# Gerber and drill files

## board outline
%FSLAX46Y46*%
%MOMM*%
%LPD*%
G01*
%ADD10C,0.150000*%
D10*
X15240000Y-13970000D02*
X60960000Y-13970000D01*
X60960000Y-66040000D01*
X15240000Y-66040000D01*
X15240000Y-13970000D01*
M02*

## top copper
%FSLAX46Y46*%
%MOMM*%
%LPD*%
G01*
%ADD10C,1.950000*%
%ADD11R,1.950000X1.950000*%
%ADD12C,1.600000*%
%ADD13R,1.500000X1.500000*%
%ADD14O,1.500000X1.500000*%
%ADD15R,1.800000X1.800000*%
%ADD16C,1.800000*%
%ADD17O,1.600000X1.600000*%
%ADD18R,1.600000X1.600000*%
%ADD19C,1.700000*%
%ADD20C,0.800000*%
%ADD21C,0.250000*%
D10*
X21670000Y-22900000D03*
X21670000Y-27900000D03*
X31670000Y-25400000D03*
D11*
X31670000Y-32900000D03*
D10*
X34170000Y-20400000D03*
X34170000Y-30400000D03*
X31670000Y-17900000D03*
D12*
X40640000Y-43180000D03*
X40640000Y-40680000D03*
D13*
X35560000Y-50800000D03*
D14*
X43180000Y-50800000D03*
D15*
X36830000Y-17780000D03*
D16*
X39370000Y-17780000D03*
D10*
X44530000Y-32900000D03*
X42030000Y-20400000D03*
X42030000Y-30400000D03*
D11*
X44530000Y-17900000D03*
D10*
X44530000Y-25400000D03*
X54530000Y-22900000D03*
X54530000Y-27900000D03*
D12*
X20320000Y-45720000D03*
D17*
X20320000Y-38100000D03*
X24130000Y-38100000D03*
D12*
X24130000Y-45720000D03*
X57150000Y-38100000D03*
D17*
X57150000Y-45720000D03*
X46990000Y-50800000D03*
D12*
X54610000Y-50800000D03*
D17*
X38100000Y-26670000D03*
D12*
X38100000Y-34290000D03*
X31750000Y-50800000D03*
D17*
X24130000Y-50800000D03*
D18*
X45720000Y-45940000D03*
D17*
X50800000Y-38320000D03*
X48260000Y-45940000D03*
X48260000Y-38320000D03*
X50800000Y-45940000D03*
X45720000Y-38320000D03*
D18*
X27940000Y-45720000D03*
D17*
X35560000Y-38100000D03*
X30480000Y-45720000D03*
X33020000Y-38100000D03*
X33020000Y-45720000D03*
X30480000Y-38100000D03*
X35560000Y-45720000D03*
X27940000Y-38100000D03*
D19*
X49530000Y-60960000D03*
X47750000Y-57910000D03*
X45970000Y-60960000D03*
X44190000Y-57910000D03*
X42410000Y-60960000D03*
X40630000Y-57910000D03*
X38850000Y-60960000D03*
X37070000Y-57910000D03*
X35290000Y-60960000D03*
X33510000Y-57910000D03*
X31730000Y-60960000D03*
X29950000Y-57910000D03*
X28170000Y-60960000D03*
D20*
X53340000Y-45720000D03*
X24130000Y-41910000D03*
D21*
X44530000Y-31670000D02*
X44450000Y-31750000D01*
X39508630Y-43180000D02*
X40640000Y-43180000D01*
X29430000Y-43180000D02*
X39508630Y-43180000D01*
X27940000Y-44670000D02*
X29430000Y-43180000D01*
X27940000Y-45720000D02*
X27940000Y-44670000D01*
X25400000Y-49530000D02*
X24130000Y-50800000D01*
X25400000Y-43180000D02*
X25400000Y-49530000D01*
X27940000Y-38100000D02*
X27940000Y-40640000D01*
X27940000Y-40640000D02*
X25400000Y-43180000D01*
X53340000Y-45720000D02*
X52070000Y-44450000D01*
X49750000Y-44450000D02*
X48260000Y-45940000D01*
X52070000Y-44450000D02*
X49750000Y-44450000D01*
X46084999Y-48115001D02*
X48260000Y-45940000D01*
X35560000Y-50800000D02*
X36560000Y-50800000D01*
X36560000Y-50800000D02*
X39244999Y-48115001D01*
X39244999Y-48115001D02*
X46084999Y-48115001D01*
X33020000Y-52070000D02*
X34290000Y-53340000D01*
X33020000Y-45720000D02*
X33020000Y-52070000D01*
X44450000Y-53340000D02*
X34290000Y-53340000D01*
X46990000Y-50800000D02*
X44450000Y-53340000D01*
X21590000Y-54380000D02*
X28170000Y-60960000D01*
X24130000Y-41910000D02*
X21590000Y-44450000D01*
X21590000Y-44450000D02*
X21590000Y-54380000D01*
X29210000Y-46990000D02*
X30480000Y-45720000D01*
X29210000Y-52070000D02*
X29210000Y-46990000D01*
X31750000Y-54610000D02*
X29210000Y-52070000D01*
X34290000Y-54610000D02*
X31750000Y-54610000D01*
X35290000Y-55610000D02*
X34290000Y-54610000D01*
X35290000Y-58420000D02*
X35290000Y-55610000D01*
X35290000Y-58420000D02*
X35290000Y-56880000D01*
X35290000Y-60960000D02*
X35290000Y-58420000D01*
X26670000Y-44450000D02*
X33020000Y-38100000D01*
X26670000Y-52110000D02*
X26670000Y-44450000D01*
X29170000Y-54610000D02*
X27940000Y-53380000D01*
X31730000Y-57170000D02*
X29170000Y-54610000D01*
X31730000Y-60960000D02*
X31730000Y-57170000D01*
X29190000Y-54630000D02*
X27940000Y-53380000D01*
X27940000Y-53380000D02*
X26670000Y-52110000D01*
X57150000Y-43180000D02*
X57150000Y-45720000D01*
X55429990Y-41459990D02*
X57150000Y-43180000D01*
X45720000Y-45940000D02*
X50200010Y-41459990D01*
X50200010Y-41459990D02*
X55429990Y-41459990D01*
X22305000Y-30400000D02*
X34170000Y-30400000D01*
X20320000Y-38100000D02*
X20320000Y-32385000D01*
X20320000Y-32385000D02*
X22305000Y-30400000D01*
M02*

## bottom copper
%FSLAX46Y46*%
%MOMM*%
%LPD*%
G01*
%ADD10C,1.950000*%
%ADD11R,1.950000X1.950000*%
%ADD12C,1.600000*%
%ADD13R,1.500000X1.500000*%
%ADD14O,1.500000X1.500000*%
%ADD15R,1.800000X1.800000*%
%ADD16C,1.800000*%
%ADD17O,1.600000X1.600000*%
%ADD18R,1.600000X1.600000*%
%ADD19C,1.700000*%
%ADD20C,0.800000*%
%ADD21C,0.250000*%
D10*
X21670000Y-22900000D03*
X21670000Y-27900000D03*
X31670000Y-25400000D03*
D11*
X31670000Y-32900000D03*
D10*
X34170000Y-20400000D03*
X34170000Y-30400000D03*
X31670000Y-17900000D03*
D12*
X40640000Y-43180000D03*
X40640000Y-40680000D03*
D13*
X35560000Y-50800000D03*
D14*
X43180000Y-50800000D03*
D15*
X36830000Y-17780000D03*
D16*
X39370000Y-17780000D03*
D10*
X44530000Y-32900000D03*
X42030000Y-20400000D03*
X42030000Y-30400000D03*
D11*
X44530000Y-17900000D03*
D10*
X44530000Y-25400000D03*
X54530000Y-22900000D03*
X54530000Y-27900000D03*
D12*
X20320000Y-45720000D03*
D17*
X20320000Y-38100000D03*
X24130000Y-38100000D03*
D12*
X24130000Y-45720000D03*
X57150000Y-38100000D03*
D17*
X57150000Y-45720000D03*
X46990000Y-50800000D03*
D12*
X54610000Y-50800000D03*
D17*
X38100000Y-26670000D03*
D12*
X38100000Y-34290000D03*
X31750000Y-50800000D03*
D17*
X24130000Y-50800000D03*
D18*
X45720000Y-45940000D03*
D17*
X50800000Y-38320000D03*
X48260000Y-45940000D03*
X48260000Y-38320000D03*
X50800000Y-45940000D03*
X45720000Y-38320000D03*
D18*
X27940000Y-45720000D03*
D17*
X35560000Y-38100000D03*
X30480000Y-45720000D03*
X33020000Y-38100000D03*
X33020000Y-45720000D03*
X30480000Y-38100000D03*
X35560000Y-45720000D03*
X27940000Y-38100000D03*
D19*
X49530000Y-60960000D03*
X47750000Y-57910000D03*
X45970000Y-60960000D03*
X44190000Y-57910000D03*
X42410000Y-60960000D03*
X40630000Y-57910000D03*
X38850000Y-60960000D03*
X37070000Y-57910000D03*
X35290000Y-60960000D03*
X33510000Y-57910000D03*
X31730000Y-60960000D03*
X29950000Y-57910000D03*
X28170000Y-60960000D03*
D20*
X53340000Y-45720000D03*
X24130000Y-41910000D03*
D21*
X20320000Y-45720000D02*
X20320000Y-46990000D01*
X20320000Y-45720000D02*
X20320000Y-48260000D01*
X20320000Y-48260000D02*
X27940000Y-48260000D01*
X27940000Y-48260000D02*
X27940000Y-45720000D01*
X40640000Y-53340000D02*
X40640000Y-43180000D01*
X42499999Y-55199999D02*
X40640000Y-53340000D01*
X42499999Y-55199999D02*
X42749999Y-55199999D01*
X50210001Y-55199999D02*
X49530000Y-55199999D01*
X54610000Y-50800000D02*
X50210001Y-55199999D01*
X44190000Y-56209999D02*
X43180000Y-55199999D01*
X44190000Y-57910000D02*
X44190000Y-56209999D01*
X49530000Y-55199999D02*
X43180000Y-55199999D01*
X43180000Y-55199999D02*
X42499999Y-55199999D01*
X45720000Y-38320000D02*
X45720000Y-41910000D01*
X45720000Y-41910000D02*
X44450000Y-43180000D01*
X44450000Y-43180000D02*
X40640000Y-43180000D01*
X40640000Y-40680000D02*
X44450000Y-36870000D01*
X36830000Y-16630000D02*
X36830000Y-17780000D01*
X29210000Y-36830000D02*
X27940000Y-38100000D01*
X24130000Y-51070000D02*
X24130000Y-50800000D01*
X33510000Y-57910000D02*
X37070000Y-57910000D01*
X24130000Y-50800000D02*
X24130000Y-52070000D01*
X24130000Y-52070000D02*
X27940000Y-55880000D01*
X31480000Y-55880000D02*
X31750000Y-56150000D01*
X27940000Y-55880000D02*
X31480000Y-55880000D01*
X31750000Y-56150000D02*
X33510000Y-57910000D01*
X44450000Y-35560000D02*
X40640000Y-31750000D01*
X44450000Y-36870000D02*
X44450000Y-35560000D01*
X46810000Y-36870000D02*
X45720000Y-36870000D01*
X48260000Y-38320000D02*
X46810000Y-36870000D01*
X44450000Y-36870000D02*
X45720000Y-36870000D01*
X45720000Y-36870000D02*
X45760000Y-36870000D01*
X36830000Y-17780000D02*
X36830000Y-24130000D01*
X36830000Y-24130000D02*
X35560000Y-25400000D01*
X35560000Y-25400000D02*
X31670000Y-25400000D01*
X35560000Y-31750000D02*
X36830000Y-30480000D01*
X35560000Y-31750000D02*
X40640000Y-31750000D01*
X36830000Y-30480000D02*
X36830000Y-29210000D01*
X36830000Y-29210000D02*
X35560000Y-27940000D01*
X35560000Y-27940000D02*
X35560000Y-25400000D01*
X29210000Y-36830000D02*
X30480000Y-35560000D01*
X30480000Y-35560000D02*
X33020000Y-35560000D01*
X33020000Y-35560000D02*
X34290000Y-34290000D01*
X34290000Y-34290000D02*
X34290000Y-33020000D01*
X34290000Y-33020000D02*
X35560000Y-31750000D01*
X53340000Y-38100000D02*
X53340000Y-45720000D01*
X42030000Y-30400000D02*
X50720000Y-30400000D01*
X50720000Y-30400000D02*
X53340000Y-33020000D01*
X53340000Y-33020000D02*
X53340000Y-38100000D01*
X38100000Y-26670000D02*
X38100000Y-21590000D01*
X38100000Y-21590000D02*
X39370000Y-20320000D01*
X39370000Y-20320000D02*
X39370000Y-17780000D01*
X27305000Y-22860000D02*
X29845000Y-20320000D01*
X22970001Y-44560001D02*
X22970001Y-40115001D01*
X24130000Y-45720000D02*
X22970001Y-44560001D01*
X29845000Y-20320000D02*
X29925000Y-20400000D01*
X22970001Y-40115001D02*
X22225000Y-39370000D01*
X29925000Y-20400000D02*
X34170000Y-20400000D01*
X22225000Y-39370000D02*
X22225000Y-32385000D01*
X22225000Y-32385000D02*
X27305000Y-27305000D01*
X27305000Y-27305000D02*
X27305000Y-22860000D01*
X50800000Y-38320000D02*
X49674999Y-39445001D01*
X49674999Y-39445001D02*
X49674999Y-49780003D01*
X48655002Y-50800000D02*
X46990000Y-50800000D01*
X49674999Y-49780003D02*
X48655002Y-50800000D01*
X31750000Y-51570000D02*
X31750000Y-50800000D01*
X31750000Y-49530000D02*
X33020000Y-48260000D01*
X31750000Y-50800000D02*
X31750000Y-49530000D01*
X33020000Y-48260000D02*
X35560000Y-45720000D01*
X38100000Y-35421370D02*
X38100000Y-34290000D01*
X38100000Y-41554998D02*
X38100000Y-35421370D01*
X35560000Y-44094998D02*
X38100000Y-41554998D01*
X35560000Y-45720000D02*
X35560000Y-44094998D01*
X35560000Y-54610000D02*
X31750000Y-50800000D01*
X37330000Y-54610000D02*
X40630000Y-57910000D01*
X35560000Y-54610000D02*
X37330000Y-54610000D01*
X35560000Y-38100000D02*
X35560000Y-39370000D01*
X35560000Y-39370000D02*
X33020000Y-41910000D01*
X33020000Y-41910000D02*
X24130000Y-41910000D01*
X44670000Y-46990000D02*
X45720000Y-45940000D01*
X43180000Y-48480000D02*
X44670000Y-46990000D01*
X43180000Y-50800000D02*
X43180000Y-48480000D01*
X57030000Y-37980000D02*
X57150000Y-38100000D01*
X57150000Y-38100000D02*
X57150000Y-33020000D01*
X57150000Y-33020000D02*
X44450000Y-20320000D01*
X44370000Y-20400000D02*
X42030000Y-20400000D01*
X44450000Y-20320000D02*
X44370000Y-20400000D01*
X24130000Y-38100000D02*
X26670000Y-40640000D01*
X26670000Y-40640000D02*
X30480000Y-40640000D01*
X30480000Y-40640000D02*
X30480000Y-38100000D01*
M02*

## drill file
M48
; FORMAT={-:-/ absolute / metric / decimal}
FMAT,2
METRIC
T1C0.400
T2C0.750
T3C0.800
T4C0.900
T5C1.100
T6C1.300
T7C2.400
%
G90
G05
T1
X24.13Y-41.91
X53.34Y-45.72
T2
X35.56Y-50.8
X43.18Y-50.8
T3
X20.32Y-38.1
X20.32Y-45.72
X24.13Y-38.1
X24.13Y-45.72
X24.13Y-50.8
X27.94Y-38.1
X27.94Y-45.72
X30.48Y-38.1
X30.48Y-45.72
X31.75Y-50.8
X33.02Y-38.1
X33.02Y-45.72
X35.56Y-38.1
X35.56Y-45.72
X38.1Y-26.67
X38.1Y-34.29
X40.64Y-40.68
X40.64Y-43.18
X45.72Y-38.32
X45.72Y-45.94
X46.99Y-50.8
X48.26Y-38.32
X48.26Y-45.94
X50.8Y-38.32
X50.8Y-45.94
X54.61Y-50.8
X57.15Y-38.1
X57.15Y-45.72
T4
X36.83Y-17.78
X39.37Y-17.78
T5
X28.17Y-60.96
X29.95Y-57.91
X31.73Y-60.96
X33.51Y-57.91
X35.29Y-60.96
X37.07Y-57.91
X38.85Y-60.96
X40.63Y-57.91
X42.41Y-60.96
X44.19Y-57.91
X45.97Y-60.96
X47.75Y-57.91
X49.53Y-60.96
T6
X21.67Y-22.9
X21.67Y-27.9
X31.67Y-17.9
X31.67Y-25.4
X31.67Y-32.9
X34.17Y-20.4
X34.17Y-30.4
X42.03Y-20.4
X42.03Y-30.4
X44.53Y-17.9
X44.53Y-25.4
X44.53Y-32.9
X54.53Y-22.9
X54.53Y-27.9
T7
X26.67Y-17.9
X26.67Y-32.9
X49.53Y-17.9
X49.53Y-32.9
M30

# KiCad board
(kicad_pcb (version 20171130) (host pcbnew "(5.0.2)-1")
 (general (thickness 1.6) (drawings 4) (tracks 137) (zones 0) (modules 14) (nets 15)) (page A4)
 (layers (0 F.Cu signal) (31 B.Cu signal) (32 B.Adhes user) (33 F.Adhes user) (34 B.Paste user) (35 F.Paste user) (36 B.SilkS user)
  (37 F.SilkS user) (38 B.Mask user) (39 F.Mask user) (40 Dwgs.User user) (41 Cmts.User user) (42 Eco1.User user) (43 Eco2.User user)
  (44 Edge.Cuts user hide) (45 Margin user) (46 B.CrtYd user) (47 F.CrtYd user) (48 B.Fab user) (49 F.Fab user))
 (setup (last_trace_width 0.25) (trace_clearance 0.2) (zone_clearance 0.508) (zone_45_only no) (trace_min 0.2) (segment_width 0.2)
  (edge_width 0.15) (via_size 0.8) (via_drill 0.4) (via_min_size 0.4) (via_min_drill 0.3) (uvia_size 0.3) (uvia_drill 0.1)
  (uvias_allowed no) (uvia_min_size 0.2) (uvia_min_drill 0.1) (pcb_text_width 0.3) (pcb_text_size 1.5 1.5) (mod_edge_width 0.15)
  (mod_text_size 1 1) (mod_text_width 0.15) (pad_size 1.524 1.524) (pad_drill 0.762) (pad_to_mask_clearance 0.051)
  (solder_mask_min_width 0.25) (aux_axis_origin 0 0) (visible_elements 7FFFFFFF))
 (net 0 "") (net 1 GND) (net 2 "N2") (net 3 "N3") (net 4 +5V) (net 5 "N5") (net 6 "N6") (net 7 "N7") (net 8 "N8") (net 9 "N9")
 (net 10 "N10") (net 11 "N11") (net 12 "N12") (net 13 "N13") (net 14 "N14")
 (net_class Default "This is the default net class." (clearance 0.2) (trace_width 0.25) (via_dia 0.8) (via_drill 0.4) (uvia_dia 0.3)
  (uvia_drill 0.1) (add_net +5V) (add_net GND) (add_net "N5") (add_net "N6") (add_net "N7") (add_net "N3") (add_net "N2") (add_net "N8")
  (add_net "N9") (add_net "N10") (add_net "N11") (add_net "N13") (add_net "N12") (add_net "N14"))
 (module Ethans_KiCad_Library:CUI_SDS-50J (layer F.Cu) (at 26.67 25.4 270)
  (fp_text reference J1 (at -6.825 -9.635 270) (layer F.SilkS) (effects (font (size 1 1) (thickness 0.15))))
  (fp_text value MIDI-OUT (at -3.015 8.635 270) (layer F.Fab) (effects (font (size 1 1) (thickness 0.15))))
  (pad E1 thru_hole circle (at -2.5 5 270) (size 1.95 1.95) (drill 1.3) (layers *.Cu *.Mask))
  (pad E2 thru_hole circle (at 2.5 5 270) (size 1.95 1.95) (drill 1.3) (layers *.Cu *.Mask))
  (pad 2 thru_hole circle (at 0 -5 270) (size 1.95 1.95) (drill 1.3) (layers *.Cu *.Mask) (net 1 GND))
  (pad 1 thru_hole rect (at 7.5 -5 270) (size 1.95 1.95) (drill 1.3) (layers *.Cu *.Mask))
  (pad 5 thru_hole circle (at -5 -7.5 270) (size 1.95 1.95) (drill 1.3) (layers *.Cu *.Mask) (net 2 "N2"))
  (pad 4 thru_hole circle (at 5 -7.5 270) (size 1.95 1.95) (drill 1.3) (layers *.Cu *.Mask) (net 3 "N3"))
  (pad None np_thru_hole circle (at 7.5 0 270) (size 2.4 2.4) (drill 2.4) (layers *.Cu *.Mask))
  (pad None np_thru_hole circle (at -7.5 0 270) (size 2.4 2.4) (drill 2.4) (layers *.Cu *.Mask))
  (pad 3 thru_hole circle (at -7.5 -5 270) (size 1.95 1.95) (drill 1.3) (layers *.Cu *.Mask)))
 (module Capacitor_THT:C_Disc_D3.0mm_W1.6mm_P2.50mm (layer F.Cu) (at 40.64 43.18 90)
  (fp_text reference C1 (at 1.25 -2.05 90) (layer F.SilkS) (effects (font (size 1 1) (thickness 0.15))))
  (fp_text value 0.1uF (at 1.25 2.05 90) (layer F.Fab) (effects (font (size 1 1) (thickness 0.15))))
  (pad 1 thru_hole circle (at 0 0 90) (size 1.6 1.6) (drill 0.8) (layers *.Cu *.Mask) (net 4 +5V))
  (pad 2 thru_hole circle (at 2.5 0 90) (size 1.6 1.6) (drill 0.8) (layers *.Cu *.Mask) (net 1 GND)))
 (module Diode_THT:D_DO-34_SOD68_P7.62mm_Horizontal (layer F.Cu) (at 35.56 50.8)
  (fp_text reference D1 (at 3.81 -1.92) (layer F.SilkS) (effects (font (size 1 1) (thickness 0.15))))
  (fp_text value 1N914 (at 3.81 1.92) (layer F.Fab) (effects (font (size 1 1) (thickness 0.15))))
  (pad 1 thru_hole rect (at 0 0) (size 1.5 1.5) (drill 0.75) (layers *.Cu *.Mask) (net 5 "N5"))
  (pad 2 thru_hole oval (at 7.62 0) (size 1.5 1.5) (drill 0.75) (layers *.Cu *.Mask) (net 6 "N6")))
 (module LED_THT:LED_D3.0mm (layer F.Cu) (at 36.83 17.78)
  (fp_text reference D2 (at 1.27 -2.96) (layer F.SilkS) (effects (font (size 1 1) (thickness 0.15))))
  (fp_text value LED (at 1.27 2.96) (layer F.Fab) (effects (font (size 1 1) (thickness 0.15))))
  (pad 1 thru_hole rect (at 0 0) (size 1.8 1.8) (drill 0.9) (layers *.Cu *.Mask) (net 1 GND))
  (pad 2 thru_hole circle (at 2.54 0) (size 1.8 1.8) (drill 0.9) (layers *.Cu *.Mask) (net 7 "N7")))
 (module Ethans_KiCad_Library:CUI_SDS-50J (layer F.Cu) (at 49.53 25.4 90)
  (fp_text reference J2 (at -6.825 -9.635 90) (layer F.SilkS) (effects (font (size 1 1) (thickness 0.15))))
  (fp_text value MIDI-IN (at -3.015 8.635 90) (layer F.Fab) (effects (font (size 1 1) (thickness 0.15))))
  (pad 3 thru_hole circle (at -7.5 -5 90) (size 1.95 1.95) (drill 1.3) (layers *.Cu *.Mask))
  (pad None np_thru_hole circle (at -7.5 0 90) (size 2.4 2.4) (drill 2.4) (layers *.Cu *.Mask))
  (pad None np_thru_hole circle (at 7.5 0 90) (size 2.4 2.4) (drill 2.4) (layers *.Cu *.Mask))
  (pad 4 thru_hole circle (at 5 -7.5 90) (size 1.95 1.95) (drill 1.3) (layers *.Cu *.Mask) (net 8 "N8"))
  (pad 5 thru_hole circle (at -5 -7.5 90) (size 1.95 1.95) (drill 1.3) (layers *.Cu *.Mask) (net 5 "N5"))
  (pad 1 thru_hole rect (at 7.5 -5 90) (size 1.95 1.95) (drill 1.3) (layers *.Cu *.Mask))
  (pad 2 thru_hole circle (at 0 -5 90) (size 1.95 1.95) (drill 1.3) (layers *.Cu *.Mask))
  (pad E2 thru_hole circle (at 2.5 5 90) (size 1.95 1.95) (drill 1.3) (layers *.Cu *.Mask))
  (pad E1 thru_hole circle (at -2.5 5 90) (size 1.95 1.95) (drill 1.3) (layers *.Cu *.Mask)))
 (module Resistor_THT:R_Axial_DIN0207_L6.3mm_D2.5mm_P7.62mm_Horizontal (layer F.Cu) (at 20.32 45.72 90)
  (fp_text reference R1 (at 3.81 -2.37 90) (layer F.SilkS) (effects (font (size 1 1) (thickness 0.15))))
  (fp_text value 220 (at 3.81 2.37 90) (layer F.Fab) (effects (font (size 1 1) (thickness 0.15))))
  (pad 1 thru_hole circle (at 0 0 90) (size 1.6 1.6) (drill 0.8) (layers *.Cu *.Mask) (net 4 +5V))
  (pad 2 thru_hole oval (at 7.62 0 90) (size 1.6 1.6) (drill 0.8) (layers *.Cu *.Mask) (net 3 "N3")))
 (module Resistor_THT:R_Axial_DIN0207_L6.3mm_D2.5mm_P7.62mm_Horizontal (layer F.Cu) (at 24.13 45.72 90)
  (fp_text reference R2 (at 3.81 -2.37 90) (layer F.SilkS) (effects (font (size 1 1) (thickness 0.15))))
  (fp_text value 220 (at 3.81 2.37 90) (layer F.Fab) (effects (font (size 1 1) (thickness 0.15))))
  (pad 2 thru_hole oval (at 7.62 0 90) (size 1.6 1.6) (drill 0.8) (layers *.Cu *.Mask) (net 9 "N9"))
  (pad 1 thru_hole circle (at 0 0 90) (size 1.6 1.6) (drill 0.8) (layers *.Cu *.Mask) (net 2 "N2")))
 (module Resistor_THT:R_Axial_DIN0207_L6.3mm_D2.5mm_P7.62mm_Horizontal (layer F.Cu) (at 57.15 38.1 270)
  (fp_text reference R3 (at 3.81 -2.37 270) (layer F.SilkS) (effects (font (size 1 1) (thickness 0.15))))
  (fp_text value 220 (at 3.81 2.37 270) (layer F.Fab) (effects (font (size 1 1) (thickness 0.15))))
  (pad 1 thru_hole circle (at 0 0 270) (size 1.6 1.6) (drill 0.8) (layers *.Cu *.Mask) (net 8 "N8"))
  (pad 2 thru_hole oval (at 7.62 0 270) (size 1.6 1.6) (drill 0.8) (layers *.Cu *.Mask) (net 6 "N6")))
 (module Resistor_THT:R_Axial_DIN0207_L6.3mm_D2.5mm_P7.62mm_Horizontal (layer F.Cu) (at 54.61 50.8 180)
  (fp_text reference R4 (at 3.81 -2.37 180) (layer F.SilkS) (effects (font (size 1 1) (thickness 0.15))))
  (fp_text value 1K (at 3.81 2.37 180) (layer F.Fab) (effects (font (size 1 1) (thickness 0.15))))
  (pad 2 thru_hole oval (at 7.62 0 180) (size 1.6 1.6) (drill 0.8) (layers *.Cu *.Mask) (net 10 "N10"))
  (pad 1 thru_hole circle (at 0 0 180) (size 1.6 1.6) (drill 0.8) (layers *.Cu *.Mask) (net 4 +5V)))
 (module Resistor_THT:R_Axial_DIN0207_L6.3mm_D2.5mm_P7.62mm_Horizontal (layer F.Cu) (at 38.1 34.29 90)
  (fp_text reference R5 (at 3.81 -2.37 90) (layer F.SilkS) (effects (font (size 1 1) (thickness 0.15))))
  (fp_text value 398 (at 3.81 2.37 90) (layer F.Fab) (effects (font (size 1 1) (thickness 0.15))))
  (pad 2 thru_hole oval (at 7.62 0 90) (size 1.6 1.6) (drill 0.8) (layers *.Cu *.Mask) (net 7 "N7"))
  (pad 1 thru_hole circle (at 0 0 90) (size 1.6 1.6) (drill 0.8) (layers *.Cu *.Mask) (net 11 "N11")))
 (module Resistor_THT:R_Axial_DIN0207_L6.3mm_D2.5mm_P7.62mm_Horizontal (layer F.Cu) (at 31.75 50.8 180)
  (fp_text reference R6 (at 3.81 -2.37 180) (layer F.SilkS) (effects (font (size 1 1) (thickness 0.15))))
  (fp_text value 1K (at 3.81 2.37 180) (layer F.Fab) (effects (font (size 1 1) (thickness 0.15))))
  (pad 1 thru_hole circle (at 0 0 180) (size 1.6 1.6) (drill 0.8) (layers *.Cu *.Mask) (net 11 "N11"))
  (pad 2 thru_hole oval (at 7.62 0 180) (size 1.6 1.6) (drill 0.8) (layers *.Cu *.Mask) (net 1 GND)))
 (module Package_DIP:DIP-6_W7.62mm (layer F.Cu) (at 45.72 45.94 90)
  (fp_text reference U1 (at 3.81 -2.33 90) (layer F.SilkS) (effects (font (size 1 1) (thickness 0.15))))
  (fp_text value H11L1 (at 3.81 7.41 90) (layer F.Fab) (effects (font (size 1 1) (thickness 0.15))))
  (pad 1 thru_hole rect (at 0 0 90) (size 1.6 1.6) (drill 0.8) (layers *.Cu *.Mask) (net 6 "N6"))
  (pad 4 thru_hole oval (at 7.62 5.08 90) (size 1.6 1.6) (drill 0.8) (layers *.Cu *.Mask) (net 10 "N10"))
  (pad 2 thru_hole oval (at 0 2.54 90) (size 1.6 1.6) (drill 0.8) (layers *.Cu *.Mask) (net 5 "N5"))
  (pad 5 thru_hole oval (at 7.62 2.54 90) (size 1.6 1.6) (drill 0.8) (layers *.Cu *.Mask) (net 1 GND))
  (pad 3 thru_hole oval (at 0 5.08 90) (size 1.6 1.6) (drill 0.8) (layers *.Cu *.Mask))
  (pad 6 thru_hole oval (at 7.62 0 90) (size 1.6 1.6) (drill 0.8) (layers *.Cu *.Mask) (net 4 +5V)))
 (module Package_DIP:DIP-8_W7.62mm (layer F.Cu) (at 27.94 45.72 90)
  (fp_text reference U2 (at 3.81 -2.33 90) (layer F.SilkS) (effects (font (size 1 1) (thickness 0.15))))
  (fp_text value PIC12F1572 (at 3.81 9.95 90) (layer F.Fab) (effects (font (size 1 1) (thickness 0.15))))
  (pad 1 thru_hole rect (at 0 0 90) (size 1.6 1.6) (drill 0.8) (layers *.Cu *.Mask) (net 4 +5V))
  (pad 5 thru_hole oval (at 7.62 7.62 90) (size 1.6 1.6) (drill 0.8) (layers *.Cu *.Mask) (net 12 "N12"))
  (pad 2 thru_hole oval (at 0 2.54 90) (size 1.6 1.6) (drill 0.8) (layers *.Cu *.Mask) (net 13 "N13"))
  (pad 6 thru_hole oval (at 7.62 5.08 90) (size 1.6 1.6) (drill 0.8) (layers *.Cu *.Mask) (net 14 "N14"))
  (pad 3 thru_hole oval (at 0 5.08 90) (size 1.6 1.6) (drill 0.8) (layers *.Cu *.Mask) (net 10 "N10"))
  (pad 7 thru_hole oval (at 7.62 2.54 90) (size 1.6 1.6) (drill 0.8) (layers *.Cu *.Mask) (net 9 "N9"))
  (pad 4 thru_hole oval (at 0 7.62 90) (size 1.6 1.6) (drill 0.8) (layers *.Cu *.Mask) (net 11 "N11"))
  (pad 8 thru_hole oval (at 7.62 0 90) (size 1.6 1.6) (drill 0.8) (layers *.Cu *.Mask) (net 1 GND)))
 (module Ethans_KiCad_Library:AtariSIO (layer F.Cu) (at 35.29 64.01)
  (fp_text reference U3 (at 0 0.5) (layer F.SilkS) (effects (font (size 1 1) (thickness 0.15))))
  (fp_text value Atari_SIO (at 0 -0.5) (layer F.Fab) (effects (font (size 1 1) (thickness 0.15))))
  (pad 13 thru_hole circle (at 14.24 -3.05) (size 1.7 1.7) (drill 1.1) (layers *.Cu *.Mask))
  (pad 12 thru_hole circle (at 12.46 -6.1) (size 1.7 1.7) (drill 1.1) (layers *.Cu *.Mask))
  (pad 11 thru_hole circle (at 10.68 -3.05) (size 1.7 1.7) (drill 1.1) (layers *.Cu *.Mask))
  (pad 10 thru_hole circle (at 8.9 -6.1) (size 1.7 1.7) (drill 1.1) (layers *.Cu *.Mask) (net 4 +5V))
  (pad 9 thru_hole circle (at 7.12 -3.05) (size 1.7 1.7) (drill 1.1) (layers *.Cu *.Mask))
  (pad 8 thru_hole circle (at 5.34 -6.1) (size 1.7 1.7) (drill 1.1) (layers *.Cu *.Mask) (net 11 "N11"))
  (pad 7 thru_hole circle (at 3.56 -3.05) (size 1.7 1.7) (drill 1.1) (layers *.Cu *.Mask))
  (pad 6 thru_hole circle (at 1.78 -6.1) (size 1.7 1.7) (drill 1.1) (layers *.Cu *.Mask) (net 1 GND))
  (pad 5 thru_hole circle (at 0 -3.05) (size 1.7 1.7) (drill 1.1) (layers *.Cu *.Mask) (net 13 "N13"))
  (pad 4 thru_hole circle (at -1.78 -6.1) (size 1.7 1.7) (drill 1.1) (layers *.Cu *.Mask) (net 1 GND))
  (pad 3 thru_hole circle (at -3.56 -3.05) (size 1.7 1.7) (drill 1.1) (layers *.Cu *.Mask) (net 14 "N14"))
  (pad 2 thru_hole circle (at -5.34 -6.1) (size 1.7 1.7) (drill 1.1) (layers *.Cu *.Mask))
  (pad 1 thru_hole circle (at -7.12 -3.05) (size 1.7 1.7) (drill 1.1) (layers *.Cu *.Mask) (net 12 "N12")))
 (gr_poly (pts (xy 15.24 13.97) (xy 60.96 13.97) (xy 60.96 66.04) (xy 15.24 66.04)) (layer Edge.Cuts) (width 0.15))
 (segment (start 44.53 31.67) (end 44.45 31.75) (width 0.25) (layer F.Cu) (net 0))
 (segment (start 20.32 45.72) (end 20.32 46.99) (width 0.25) (layer B.Cu) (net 4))
 (segment (start 20.32 45.72) (end 20.32 48.26) (width 0.25) (layer B.Cu) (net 4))
 (segment (start 20.32 48.26) (end 27.94 48.26) (width 0.25) (layer B.Cu) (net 4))
 (segment (start 27.94 48.26) (end 27.94 45.72) (width 0.25) (layer B.Cu) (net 4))
 (segment (start 39.50863 43.18) (end 40.64 43.18) (width 0.25) (layer F.Cu) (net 4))
 (segment (start 29.43 43.18) (end 39.50863 43.18) (width 0.25) (layer F.Cu) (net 4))
 (segment (start 27.94 44.67) (end 29.43 43.18) (width 0.25) (layer F.Cu) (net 4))
 (segment (start 27.94 45.72) (end 27.94 44.67) (width 0.25) (layer F.Cu) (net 4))
 (segment (start 40.64 53.34) (end 40.64 43.18) (width 0.25) (layer B.Cu) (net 4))
 (segment (start 42.499999 55.199999) (end 40.64 53.34) (width 0.25) (layer B.Cu) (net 4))
 (segment (start 42.499999 55.199999) (end 42.749999 55.199999) (width 0.25) (layer B.Cu) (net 4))
 (segment (start 50.210001 55.199999) (end 49.53 55.199999) (width 0.25) (layer B.Cu) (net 4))
 (segment (start 54.61 50.8) (end 50.210001 55.199999) (width 0.25) (layer B.Cu) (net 4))
 (segment (start 44.19 56.209999) (end 43.18 55.199999) (width 0.25) (layer B.Cu) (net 4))
 (segment (start 44.19 57.91) (end 44.19 56.209999) (width 0.25) (layer B.Cu) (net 4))
 (segment (start 49.53 55.199999) (end 43.18 55.199999) (width 0.25) (layer B.Cu) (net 4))
 (segment (start 43.18 55.199999) (end 42.499999 55.199999) (width 0.25) (layer B.Cu) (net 4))
 (segment (start 45.72 38.32) (end 45.72 41.91) (width 0.25) (layer B.Cu) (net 4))
 (segment (start 45.72 41.91) (end 44.45 43.18) (width 0.25) (layer B.Cu) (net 4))
 (segment (start 44.45 43.18) (end 40.64 43.18) (width 0.25) (layer B.Cu) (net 4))
 (segment (start 40.64 40.68) (end 44.45 36.87) (width 0.25) (layer B.Cu) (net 1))
 (segment (start 36.83 16.63) (end 36.83 17.78) (width 0.25) (layer B.Cu) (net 1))
 (segment (start 29.21 36.83) (end 27.94 38.1) (width 0.25) (layer B.Cu) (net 1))
 (segment (start 24.13 51.07) (end 24.13 50.8) (width 0.25) (layer B.Cu) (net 1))
 (segment (start 33.51 57.91) (end 37.07 57.91) (width 0.25) (layer B.Cu) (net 1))
 (segment (start 25.4 49.53) (end 24.13 50.8) (width 0.25) (layer F.Cu) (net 1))
 (segment (start 25.4 43.18) (end 25.4 49.53) (width 0.25) (layer F.Cu) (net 1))
 (segment (start 27.94 38.1) (end 27.94 40.64) (width 0.25) (layer F.Cu) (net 1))
 (segment (start 27.94 40.64) (end 25.4 43.18) (width 0.25) (layer F.Cu) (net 1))
 (segment (start 24.13 50.8) (end 24.13 52.07) (width 0.25) (layer B.Cu) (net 1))
 (segment (start 24.13 52.07) (end 27.94 55.88) (width 0.25) (layer B.Cu) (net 1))
 (segment (start 31.48 55.88) (end 31.75 56.15) (width 0.25) (layer B.Cu) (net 1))
 (segment (start 27.94 55.88) (end 31.48 55.88) (width 0.25) (layer B.Cu) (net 1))
 (segment (start 31.75 56.15) (end 33.51 57.91) (width 0.25) (layer B.Cu) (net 1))
 (segment (start 44.45 35.56) (end 40.64 31.75) (width 0.25) (layer B.Cu) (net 1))
 (segment (start 44.45 36.87) (end 44.45 35.56) (width 0.25) (layer B.Cu) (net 1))
 (segment (start 46.81 36.87) (end 45.72 36.87) (width 0.25) (layer B.Cu) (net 1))
 (segment (start 48.26 38.32) (end 46.81 36.87) (width 0.25) (layer B.Cu) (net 1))
 (segment (start 44.45 36.87) (end 45.72 36.87) (width 0.25) (layer B.Cu) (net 1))
 (segment (start 45.72 36.87) (end 45.76 36.87) (width 0.25) (layer B.Cu) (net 1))
 (segment (start 36.83 17.78) (end 36.83 24.13) (width 0.25) (layer B.Cu) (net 1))
 (segment (start 36.83 24.13) (end 35.56 25.4) (width 0.25) (layer B.Cu) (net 1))
 (segment (start 35.56 25.4) (end 31.67 25.4) (width 0.25) (layer B.Cu) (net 1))
 (segment (start 35.56 31.75) (end 36.83 30.48) (width 0.25) (layer B.Cu) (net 1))
 (segment (start 35.56 31.75) (end 40.64 31.75) (width 0.25) (layer B.Cu) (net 1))
 (segment (start 36.83 30.48) (end 36.83 29.21) (width 0.25) (layer B.Cu) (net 1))
 (segment (start 36.83 29.21) (end 35.56 27.94) (width 0.25) (layer B.Cu) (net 1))
 (segment (start 35.56 27.94) (end 35.56 25.4) (width 0.25) (layer B.Cu) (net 1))
 (segment (start 29.21 36.83) (end 30.48 35.56) (width 0.25) (layer B.Cu) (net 1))
 (segment (start 30.48 35.56) (end 33.02 35.56) (width 0.25) (layer B.Cu) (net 1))
 (segment (start 33.02 35.56) (end 34.29 34.29) (width 0.25) (layer B.Cu) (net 1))
 (segment (start 34.29 34.29) (end 34.29 33.02) (width 0.25) (layer B.Cu) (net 1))
 (segment (start 34.29 33.02) (end 35.56 31.75) (width 0.25) (layer B.Cu) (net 1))
 (segment (start 53.34 38.1) (end 53.34 45.72) (width 0.25) (layer B.Cu) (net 5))
 (via (at 53.34 45.72) (size 0.8) (drill 0.4) (layers F.Cu B.Cu) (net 5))
 (segment (start 53.34 45.72) (end 52.07 44.45) (width 0.25) (layer F.Cu) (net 5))
 (segment (start 49.75 44.45) (end 48.26 45.94) (width 0.25) (layer F.Cu) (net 5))
 (segment (start 52.07 44.45) (end 49.75 44.45) (width 0.25) (layer F.Cu) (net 5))
 (segment (start 46.084999 48.115001) (end 48.26 45.94) (width 0.25) (layer F.Cu) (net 5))
 (segment (start 35.56 50.8) (end 36.56 50.8) (width 0.25) (layer F.Cu) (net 5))
 (segment (start 36.56 50.8) (end 39.244999 48.115001) (width 0.25) (layer F.Cu) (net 5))
 (segment (start 39.244999 48.115001) (end 46.084999 48.115001) (width 0.25) (layer F.Cu) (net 5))
 (segment (start 42.03 30.4) (end 50.72 30.4) (width 0.25) (layer B.Cu) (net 5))
 (segment (start 50.72 30.4) (end 53.34 33.02) (width 0.25) (layer B.Cu) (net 5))
 (segment (start 53.34 33.02) (end 53.34 38.1) (width 0.25) (layer B.Cu) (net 5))
 (segment (start 38.1 26.67) (end 38.1 21.59) (width 0.25) (layer B.Cu) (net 7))
 (segment (start 38.1 21.59) (end 39.37 20.32) (width 0.25) (layer B.Cu) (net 7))
 (segment (start 39.37 20.32) (end 39.37 17.78) (width 0.25) (layer B.Cu) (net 7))
 (segment (start 27.305 22.86) (end 29.845 20.32) (width 0.25) (layer B.Cu) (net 2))
 (segment (start 22.970001 44.560001) (end 22.970001 40.115001) (width 0.25) (layer B.Cu) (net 2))
 (segment (start 24.13 45.72) (end 22.970001 44.560001) (width 0.25) (layer B.Cu) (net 2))
 (segment (start 29.845 20.32) (end 29.925 20.4) (width 0.25) (layer B.Cu) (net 2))
 (segment (start 22.970001 40.115001) (end 22.225 39.37) (width 0.25) (layer B.Cu) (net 2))
 (segment (start 29.925 20.4) (end 34.17 20.4) (width 0.25) (layer B.Cu) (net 2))
 (segment (start 22.225 39.37) (end 22.225 32.385) (width 0.25) (layer B.Cu) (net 2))
 (segment (start 22.225 32.385) (end 27.305 27.305) (width 0.25) (layer B.Cu) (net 2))
 (segment (start 27.305 27.305) (end 27.305 22.86) (width 0.25) (layer B.Cu) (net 2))
 (segment (start 33.02 52.07) (end 34.29 53.34) (width 0.25) (layer F.Cu) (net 10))
 (segment (start 50.8 38.32) (end 49.674999 39.445001) (width 0.25) (layer B.Cu) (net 10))
 (segment (start 49.674999 39.445001) (end 49.674999 49.780003) (width 0.25) (layer B.Cu) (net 10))
 (segment (start 33.02 45.72) (end 33.02 52.07) (width 0.25) (layer F.Cu) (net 10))
 (segment (start 44.45 53.34) (end 34.29 53.34) (width 0.25) (layer F.Cu) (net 10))
 (segment (start 46.99 50.8) (end 44.45 53.34) (width 0.25) (layer F.Cu) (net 10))
 (segment (start 48.655002 50.8) (end 46.99 50.8) (width 0.25) (layer B.Cu) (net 10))
 (segment (start 49.674999 49.780003) (end 48.655002 50.8) (width 0.25) (layer B.Cu) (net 10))
 (segment (start 31.75 51.57) (end 31.75 50.8) (width 0.25) (layer B.Cu) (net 11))
 (segment (start 31.75 49.53) (end 33.02 48.26) (width 0.25) (layer B.Cu) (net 11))
 (segment (start 31.75 50.8) (end 31.75 49.53) (width 0.25) (layer B.Cu) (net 11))
 (segment (start 33.02 48.26) (end 35.56 45.72) (width 0.25) (layer B.Cu) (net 11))
 (segment (start 38.1 35.42137) (end 38.1 34.29) (width 0.25) (layer B.Cu) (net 11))
 (segment (start 38.1 41.554998) (end 38.1 35.42137) (width 0.25) (layer B.Cu) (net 11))
 (segment (start 35.56 44.094998) (end 38.1 41.554998) (width 0.25) (layer B.Cu) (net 11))
 (segment (start 35.56 45.72) (end 35.56 44.094998) (width 0.25) (layer B.Cu) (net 11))
 (segment (start 35.56 54.61) (end 31.75 50.8) (width 0.25) (layer B.Cu) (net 11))
 (segment (start 37.33 54.61) (end 40.63 57.91) (width 0.25) (layer B.Cu) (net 11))
 (segment (start 35.56 54.61) (end 37.33 54.61) (width 0.25) (layer B.Cu) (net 11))
 (segment (start 35.56 38.1) (end 35.56 39.37) (width 0.25) (layer B.Cu) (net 12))
 (segment (start 35.56 39.37) (end 33.02 41.91) (width 0.25) (layer B.Cu) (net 12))
 (via (at 24.13 41.91) (size 0.8) (drill 0.4) (layers F.Cu B.Cu) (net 12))
 (segment (start 33.02 41.91) (end 24.13 41.91) (width 0.25) (layer B.Cu) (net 12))
 (segment (start 21.59 54.38) (end 28.17 60.96) (width 0.25) (layer F.Cu) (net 12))
 (segment (start 24.13 41.91) (end 21.59 44.45) (width 0.25) (layer F.Cu) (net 12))
 (segment (start 21.59 44.45) (end 21.59 54.38) (width 0.25) (layer F.Cu) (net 12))
 (segment (start 29.21 46.99) (end 30.48 45.72) (width 0.25) (layer F.Cu) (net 13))
 (segment (start 29.21 52.07) (end 29.21 46.99) (width 0.25) (layer F.Cu) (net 13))
 (segment (start 31.75 54.61) (end 29.21 52.07) (width 0.25) (layer F.Cu) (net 13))
 (segment (start 34.29 54.61) (end 31.75 54.61) (width 0.25) (layer F.Cu) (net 13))
 (segment (start 35.29 55.61) (end 34.29 54.61) (width 0.25) (layer F.Cu) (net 13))
 (segment (start 35.29 58.42) (end 35.29 55.61) (width 0.25) (layer F.Cu) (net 13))
 (segment (start 35.29 58.42) (end 35.29 56.88) (width 0.25) (layer F.Cu) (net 13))
 (segment (start 35.29 60.96) (end 35.29 58.42) (width 0.25) (layer F.Cu) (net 13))
 (segment (start 26.67 44.45) (end 33.02 38.1) (width 0.25) (layer F.Cu) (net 14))
 (segment (start 26.67 52.11) (end 26.67 44.45) (width 0.25) (layer F.Cu) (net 14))
 (segment (start 29.17 54.61) (end 27.94 53.38) (width 0.25) (layer F.Cu) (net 14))
 (segment (start 31.73 57.17) (end 29.17 54.61) (width 0.25) (layer F.Cu) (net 14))
 (segment (start 31.73 60.96) (end 31.73 57.17) (width 0.25) (layer F.Cu) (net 14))
 (segment (start 29.19 54.63) (end 27.94 53.38) (width 0.25) (layer F.Cu) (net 14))
 (segment (start 27.94 53.38) (end 26.67 52.11) (width 0.25) (layer F.Cu) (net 14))
 (segment (start 44.67 46.99) (end 45.72 45.94) (width 0.25) (layer B.Cu) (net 6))
 (segment (start 57.15 43.18) (end 57.15 45.72) (width 0.25) (layer F.Cu) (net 6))
 (segment (start 55.42999 41.45999) (end 57.15 43.18) (width 0.25) (layer F.Cu) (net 6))
 (segment (start 45.72 45.94) (end 50.20001 41.45999) (width 0.25) (layer F.Cu) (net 6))
 (segment (start 50.20001 41.45999) (end 55.42999 41.45999) (width 0.25) (layer F.Cu) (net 6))
 (segment (start 43.18 48.48) (end 44.67 46.99) (width 0.25) (layer B.Cu) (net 6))
 (segment (start 43.18 50.8) (end 43.18 48.48) (width 0.25) (layer B.Cu) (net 6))
 (segment (start 22.305 30.4) (end 34.17 30.4) (width 0.25) (layer F.Cu) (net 3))
 (segment (start 20.32 38.1) (end 20.32 32.385) (width 0.25) (layer F.Cu) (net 3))
 (segment (start 20.32 32.385) (end 22.305 30.4) (width 0.25) (layer F.Cu) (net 3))
 (segment (start 57.03 37.98) (end 57.15 38.1) (width 0.25) (layer B.Cu) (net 8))
 (segment (start 57.15 38.1) (end 57.15 33.02) (width 0.25) (layer B.Cu) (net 8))
 (segment (start 57.15 33.02) (end 44.45 20.32) (width 0.25) (layer B.Cu) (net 8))
 (segment (start 44.37 20.4) (end 42.03 20.4) (width 0.25) (layer B.Cu) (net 8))
 (segment (start 44.45 20.32) (end 44.37 20.4) (width 0.25) (layer B.Cu) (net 8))
 (segment (start 24.13 38.1) (end 26.67 40.64) (width 0.25) (layer B.Cu) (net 9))
 (segment (start 26.67 40.64) (end 30.48 40.64) (width 0.25) (layer B.Cu) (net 9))
 (segment (start 30.48 40.64) (end 30.48 38.1) (width 0.25) (layer B.Cu) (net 9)))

